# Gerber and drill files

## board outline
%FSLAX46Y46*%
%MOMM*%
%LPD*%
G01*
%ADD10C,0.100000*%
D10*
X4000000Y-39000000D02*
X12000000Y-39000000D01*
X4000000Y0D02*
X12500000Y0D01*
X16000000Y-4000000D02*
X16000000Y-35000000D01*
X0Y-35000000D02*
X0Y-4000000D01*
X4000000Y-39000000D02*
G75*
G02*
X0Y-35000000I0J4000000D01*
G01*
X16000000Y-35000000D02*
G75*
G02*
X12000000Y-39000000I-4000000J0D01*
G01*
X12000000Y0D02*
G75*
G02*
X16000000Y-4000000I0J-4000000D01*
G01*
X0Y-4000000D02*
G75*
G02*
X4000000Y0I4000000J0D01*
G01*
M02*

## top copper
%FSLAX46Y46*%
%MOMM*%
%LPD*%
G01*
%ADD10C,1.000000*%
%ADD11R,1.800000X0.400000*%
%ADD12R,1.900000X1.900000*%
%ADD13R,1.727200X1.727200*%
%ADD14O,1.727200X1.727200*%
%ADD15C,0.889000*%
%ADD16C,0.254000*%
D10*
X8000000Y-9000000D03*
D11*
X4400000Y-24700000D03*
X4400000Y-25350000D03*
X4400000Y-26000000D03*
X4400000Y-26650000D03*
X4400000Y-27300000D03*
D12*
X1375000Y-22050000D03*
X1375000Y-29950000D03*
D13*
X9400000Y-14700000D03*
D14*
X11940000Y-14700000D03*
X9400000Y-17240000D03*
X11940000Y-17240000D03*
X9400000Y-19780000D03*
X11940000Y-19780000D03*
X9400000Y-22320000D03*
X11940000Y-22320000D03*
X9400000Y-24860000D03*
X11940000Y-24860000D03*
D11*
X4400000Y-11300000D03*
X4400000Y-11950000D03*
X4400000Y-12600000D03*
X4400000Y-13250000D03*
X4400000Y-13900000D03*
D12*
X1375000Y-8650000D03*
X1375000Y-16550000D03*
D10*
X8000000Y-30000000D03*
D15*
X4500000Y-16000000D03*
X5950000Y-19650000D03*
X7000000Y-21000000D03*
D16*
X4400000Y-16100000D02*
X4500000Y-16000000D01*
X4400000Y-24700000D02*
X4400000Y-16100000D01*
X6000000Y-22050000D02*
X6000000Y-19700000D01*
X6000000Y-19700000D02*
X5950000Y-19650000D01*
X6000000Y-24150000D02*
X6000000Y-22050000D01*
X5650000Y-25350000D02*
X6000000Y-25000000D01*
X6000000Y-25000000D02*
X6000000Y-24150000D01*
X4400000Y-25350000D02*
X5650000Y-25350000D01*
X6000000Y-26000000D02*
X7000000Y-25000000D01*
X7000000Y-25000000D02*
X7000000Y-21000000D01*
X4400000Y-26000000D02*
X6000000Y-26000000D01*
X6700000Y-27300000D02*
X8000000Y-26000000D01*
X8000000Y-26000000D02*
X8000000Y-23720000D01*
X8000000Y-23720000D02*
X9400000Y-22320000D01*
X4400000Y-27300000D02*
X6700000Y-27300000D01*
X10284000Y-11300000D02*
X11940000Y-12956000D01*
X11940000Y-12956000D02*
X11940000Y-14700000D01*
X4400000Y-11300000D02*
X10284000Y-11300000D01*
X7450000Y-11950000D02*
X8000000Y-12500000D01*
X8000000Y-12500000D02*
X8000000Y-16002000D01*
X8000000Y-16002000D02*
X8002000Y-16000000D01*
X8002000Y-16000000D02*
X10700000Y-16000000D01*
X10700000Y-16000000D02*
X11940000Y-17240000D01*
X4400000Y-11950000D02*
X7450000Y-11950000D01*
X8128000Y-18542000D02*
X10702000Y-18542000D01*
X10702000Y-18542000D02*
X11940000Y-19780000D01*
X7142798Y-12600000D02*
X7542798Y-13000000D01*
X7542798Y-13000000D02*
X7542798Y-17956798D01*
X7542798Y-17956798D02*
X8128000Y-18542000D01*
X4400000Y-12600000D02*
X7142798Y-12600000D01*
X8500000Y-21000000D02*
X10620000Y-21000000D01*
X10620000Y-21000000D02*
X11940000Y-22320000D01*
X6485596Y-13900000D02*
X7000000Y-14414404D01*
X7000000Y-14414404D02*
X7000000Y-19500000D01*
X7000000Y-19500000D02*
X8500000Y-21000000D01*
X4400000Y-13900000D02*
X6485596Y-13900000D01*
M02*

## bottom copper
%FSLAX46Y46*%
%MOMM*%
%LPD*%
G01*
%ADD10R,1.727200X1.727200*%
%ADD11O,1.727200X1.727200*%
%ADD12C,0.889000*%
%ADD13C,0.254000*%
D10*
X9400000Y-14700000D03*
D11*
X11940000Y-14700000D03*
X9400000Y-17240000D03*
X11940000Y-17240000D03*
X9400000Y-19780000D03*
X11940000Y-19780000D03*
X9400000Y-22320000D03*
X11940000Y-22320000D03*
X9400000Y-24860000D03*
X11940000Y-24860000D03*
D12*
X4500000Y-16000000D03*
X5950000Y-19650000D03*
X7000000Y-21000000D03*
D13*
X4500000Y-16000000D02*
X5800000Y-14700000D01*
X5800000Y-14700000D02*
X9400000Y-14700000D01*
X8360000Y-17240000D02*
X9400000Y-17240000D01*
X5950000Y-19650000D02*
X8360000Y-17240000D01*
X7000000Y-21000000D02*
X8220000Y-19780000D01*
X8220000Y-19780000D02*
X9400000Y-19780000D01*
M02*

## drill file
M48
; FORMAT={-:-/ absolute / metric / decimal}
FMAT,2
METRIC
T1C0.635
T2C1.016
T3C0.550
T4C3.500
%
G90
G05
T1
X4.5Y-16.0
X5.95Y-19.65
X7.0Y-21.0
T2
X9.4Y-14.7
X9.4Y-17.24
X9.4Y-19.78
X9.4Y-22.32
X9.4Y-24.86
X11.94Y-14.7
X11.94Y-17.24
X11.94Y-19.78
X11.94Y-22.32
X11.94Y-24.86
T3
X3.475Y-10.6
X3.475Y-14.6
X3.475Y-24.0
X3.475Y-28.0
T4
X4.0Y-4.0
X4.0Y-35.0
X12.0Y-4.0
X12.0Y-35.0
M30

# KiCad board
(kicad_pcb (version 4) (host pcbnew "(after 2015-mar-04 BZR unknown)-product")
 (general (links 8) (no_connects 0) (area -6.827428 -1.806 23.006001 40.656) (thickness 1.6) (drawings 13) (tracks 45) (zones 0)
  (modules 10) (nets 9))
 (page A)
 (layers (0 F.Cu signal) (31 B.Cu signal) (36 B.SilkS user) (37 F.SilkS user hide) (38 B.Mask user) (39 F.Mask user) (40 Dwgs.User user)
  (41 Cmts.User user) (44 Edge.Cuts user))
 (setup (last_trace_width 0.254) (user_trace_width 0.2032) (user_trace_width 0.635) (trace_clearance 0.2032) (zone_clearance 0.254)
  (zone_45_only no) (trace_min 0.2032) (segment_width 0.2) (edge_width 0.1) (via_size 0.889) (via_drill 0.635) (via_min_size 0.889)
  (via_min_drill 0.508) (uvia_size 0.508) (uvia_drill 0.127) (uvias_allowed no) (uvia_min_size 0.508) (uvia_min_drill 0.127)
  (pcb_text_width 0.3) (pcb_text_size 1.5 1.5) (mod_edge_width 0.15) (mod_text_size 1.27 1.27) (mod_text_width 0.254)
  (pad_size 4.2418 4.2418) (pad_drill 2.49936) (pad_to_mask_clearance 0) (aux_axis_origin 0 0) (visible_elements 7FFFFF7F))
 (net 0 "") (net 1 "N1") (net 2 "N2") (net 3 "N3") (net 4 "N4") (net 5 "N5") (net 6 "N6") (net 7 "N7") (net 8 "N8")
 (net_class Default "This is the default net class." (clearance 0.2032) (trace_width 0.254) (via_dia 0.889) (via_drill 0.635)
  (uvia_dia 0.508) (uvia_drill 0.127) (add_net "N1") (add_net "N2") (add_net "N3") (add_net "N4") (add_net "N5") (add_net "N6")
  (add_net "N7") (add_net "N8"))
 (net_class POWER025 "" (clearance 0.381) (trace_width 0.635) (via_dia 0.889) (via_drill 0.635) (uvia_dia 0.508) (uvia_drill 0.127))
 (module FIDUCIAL (layer F.Cu) (at 8 9)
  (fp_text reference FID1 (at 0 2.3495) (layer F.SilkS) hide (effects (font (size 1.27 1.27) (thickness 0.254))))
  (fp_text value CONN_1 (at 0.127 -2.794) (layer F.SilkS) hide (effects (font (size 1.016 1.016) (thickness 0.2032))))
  (pad 1 smd circle (at 0 0) (size 1 1) (layers F.Cu F.Mask) (solder_mask_margin 1) (clearance 1)))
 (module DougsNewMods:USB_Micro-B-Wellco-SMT (layer F.Cu) (at 4 26 270)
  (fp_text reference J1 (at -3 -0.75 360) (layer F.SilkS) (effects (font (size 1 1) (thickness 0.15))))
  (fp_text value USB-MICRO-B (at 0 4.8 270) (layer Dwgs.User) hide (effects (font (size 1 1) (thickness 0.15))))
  (pad 1 smd rect (at -1.3 -0.4 270) (size 0.4 1.8) (layers F.Cu F.Mask) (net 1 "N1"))
  (pad 2 smd rect (at -0.65 -0.4 270) (size 0.4 1.8) (layers F.Cu F.Mask) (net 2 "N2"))
  (pad 3 smd rect (at 0 -0.4 270) (size 0.4 1.8) (layers F.Cu F.Mask) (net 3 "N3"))
  (pad 4 smd rect (at 0.65 -0.4 270) (size 0.4 1.8) (layers F.Cu F.Mask))
  (pad 5 smd rect (at 1.3 -0.4 270) (size 0.4 1.8) (layers F.Cu F.Mask) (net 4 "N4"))
  (pad "" np_thru_hole circle (at -2 0.525) (size 0.55 0.55) (drill 0.55) (layers *.Cu *.Mask F.SilkS))
  (pad "" np_thru_hole circle (at 2 0.525) (size 0.55 0.55) (drill oval 0.55) (layers *.Cu *.Mask F.SilkS))
  (pad 7 smd rect (at -3.95 2.625) (size 1.9 1.9) (layers F.Cu F.Mask))
  (pad 6 smd rect (at 3.95 2.625) (size 1.9 1.9) (layers F.Cu F.Mask)))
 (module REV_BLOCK (layer B.Cu) (at 13.15 10.8)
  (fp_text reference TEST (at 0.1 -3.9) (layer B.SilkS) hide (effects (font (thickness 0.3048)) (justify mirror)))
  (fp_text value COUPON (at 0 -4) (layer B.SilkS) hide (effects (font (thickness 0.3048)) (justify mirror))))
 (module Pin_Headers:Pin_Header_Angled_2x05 (layer F.Cu) (at 9.4 14.7)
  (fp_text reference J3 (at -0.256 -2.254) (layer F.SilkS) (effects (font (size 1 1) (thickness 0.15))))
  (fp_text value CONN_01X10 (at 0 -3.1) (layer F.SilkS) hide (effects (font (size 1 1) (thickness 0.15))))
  (pad 1 thru_hole rect (at 0 0) (size 1.7272 1.7272) (drill 1.016) (layers *.Cu *.Mask F.SilkS) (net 1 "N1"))
  (pad 2 thru_hole oval (at 2.54 0) (size 1.7272 1.7272) (drill 1.016) (layers *.Cu *.Mask F.SilkS) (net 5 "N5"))
  (pad 3 thru_hole oval (at 0 2.54) (size 1.7272 1.7272) (drill 1.016) (layers *.Cu *.Mask F.SilkS) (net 2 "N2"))
  (pad 4 thru_hole oval (at 2.54 2.54) (size 1.7272 1.7272) (drill 1.016) (layers *.Cu *.Mask F.SilkS) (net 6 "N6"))
  (pad 5 thru_hole oval (at 0 5.08) (size 1.7272 1.7272) (drill 1.016) (layers *.Cu *.Mask F.SilkS) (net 3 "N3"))
  (pad 6 thru_hole oval (at 2.54 5.08) (size 1.7272 1.7272) (drill 1.016) (layers *.Cu *.Mask F.SilkS) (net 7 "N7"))
  (pad 7 thru_hole oval (at 0 7.62) (size 1.7272 1.7272) (drill 1.016) (layers *.Cu *.Mask F.SilkS) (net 4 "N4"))
  (pad 8 thru_hole oval (at 2.54 7.62) (size 1.7272 1.7272) (drill 1.016) (layers *.Cu *.Mask F.SilkS) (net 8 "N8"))
  (pad 9 thru_hole oval (at 0 10.16) (size 1.7272 1.7272) (drill 1.016) (layers *.Cu *.Mask F.SilkS))
  (pad 10 thru_hole oval (at 2.54 10.16) (size 1.7272 1.7272) (drill 1.016) (layers *.Cu *.Mask F.SilkS)))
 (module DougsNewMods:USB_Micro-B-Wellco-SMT (layer F.Cu) (at 4 12.6 270) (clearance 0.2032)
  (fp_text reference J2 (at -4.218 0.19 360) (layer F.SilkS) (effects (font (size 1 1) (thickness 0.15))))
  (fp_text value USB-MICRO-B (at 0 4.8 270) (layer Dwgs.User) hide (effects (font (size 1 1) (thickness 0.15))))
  (pad 1 smd rect (at -1.3 -0.4 270) (size 0.4 1.8) (layers F.Cu F.Mask) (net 5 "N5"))
  (pad 2 smd rect (at -0.65 -0.4 270) (size 0.4 1.8) (layers F.Cu F.Mask) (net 6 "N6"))
  (pad 3 smd rect (at 0 -0.4 270) (size 0.4 1.8) (layers F.Cu F.Mask) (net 7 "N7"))
  (pad 4 smd rect (at 0.65 -0.4 270) (size 0.4 1.8) (layers F.Cu F.Mask))
  (pad 5 smd rect (at 1.3 -0.4 270) (size 0.4 1.8) (layers F.Cu F.Mask) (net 8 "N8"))
  (pad "" np_thru_hole circle (at -2 0.525) (size 0.55 0.55) (drill 0.55) (layers *.Cu *.Mask F.SilkS))
  (pad "" np_thru_hole circle (at 2 0.525) (size 0.55 0.55) (drill oval 0.55) (layers *.Cu *.Mask F.SilkS))
  (pad 7 smd rect (at -3.95 2.625) (size 1.9 1.9) (layers F.Cu F.Mask))
  (pad 6 smd rect (at 3.95 2.625) (size 1.9 1.9) (layers F.Cu F.Mask)))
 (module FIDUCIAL (layer F.Cu) (at 8 30)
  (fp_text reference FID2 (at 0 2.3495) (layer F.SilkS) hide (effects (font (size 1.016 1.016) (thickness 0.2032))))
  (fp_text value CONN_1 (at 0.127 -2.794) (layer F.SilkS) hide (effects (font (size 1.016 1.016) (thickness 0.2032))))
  (pad 1 smd circle (at 0 0) (size 1 1) (layers F.Cu F.Mask) (solder_mask_margin 1) (clearance 1)))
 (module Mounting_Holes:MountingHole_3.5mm (layer F.Cu) (at 4 4)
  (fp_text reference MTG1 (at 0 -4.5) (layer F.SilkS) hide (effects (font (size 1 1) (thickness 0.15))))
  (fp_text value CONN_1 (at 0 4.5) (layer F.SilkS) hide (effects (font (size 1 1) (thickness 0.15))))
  (pad 1 np_thru_hole circle (at 0 0) (size 3.5 3.5) (drill 3.5) (layers *.Cu *.Mask F.SilkS)))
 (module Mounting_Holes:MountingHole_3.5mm (layer F.Cu) (at 12 4)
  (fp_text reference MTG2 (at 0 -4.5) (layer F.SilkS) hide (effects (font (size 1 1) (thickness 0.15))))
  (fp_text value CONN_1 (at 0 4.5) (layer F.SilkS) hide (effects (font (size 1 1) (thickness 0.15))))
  (pad 1 np_thru_hole circle (at 0 0) (size 3.5 3.5) (drill 3.5) (layers *.Cu *.Mask F.SilkS)))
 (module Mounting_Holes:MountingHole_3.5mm (layer F.Cu) (at 4 35)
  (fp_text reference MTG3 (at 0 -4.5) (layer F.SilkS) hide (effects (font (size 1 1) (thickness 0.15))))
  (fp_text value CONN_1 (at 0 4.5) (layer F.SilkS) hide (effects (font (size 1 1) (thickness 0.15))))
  (pad 1 np_thru_hole circle (at 0 0) (size 3.5 3.5) (drill 3.5) (layers *.Cu *.Mask F.SilkS)))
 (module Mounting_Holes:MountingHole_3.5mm (layer F.Cu) (at 12 35)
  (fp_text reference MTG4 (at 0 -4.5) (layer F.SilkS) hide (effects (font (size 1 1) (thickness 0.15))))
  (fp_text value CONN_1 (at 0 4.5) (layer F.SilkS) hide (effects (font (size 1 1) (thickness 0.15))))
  (pad 1 np_thru_hole circle (at 0 0) (size 3.5 3.5) (drill 3.5) (layers *.Cu *.Mask F.SilkS)))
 (gr_line (start 4 39) (end 12 39) (angle 90) (layer Edge.Cuts) (width 0.1))
 (gr_line (start 4 0) (end 12.5 0) (angle 90) (layer Edge.Cuts) (width 0.1))
 (gr_line (start 16 4) (end 16 35) (angle 90) (layer Edge.Cuts) (width 0.1))
 (gr_line (start 0 35) (end 0 4) (angle 90) (layer Edge.Cuts) (width 0.1))
 (gr_arc (start 4 35) (end 4 39) (angle 90) (layer Edge.Cuts) (width 0.1))
 (gr_arc (start 12 35) (end 16 35) (angle 90) (layer Edge.Cuts) (width 0.1))
 (gr_arc (start 12 4) (end 12 0) (angle 90) (layer Edge.Cuts) (width 0.1))
 (gr_arc (start 4 4) (end 0 4) (angle 90) (layer Edge.Cuts) (width 0.1))
 (segment (start 4.4 16.1) (end 4.5 16) (width 0.254) (layer F.Cu) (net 1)) (via (at 4.5 16) (size 0.889) (layers F.Cu B.Cu) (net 1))
 (segment (start 4.5 16) (end 5.8 14.7) (width 0.254) (layer B.Cu) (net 1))
 (segment (start 5.8 14.7) (end 9.4 14.7) (width 0.254) (layer B.Cu) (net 1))
 (segment (start 4.4 24.7) (end 4.4 16.1) (width 0.254) (layer F.Cu) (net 1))
 (segment (start 6 22.05) (end 6 19.7) (width 0.254) (layer F.Cu) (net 2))
 (segment (start 8.36 17.24) (end 9.4 17.24) (width 0.254) (layer B.Cu) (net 2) (status 800000))
 (segment (start 5.95 19.65) (end 8.36 17.24) (width 0.254) (layer B.Cu) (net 2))
 (via (at 5.95 19.65) (size 0.889) (layers F.Cu B.Cu) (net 2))
 (segment (start 6 19.7) (end 5.95 19.65) (width 0.254) (layer F.Cu) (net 2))
 (segment (start 6 24.15) (end 6 22.05) (width 0.254) (layer F.Cu) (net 2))
 (segment (start 5.65 25.35) (end 6 25) (width 0.254) (layer F.Cu) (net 2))
 (segment (start 6 25) (end 6 24.15) (width 0.254) (layer F.Cu) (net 2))
 (segment (start 4.4 25.35) (end 5.65 25.35) (width 0.254) (layer F.Cu) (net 2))
 (segment (start 6 26) (end 7 25) (width 0.254) (layer F.Cu) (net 3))
 (segment (start 7 25) (end 7 21) (width 0.254) (layer F.Cu) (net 3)) (via (at 7 21) (size 0.889) (layers F.Cu B.Cu) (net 3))
 (segment (start 7 21) (end 8.22 19.78) (width 0.254) (layer B.Cu) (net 3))
 (segment (start 8.22 19.78) (end 9.4 19.78) (width 0.254) (layer B.Cu) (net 3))
 (segment (start 4.4 26) (end 6 26) (width 0.254) (layer F.Cu) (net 3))
 (segment (start 6.7 27.3) (end 8 26) (width 0.254) (layer F.Cu) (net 4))
 (segment (start 8 26) (end 8 23.72) (width 0.254) (layer F.Cu) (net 4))
 (segment (start 8 23.72) (end 9.4 22.32) (width 0.254) (layer F.Cu) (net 4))
 (segment (start 4.4 27.3) (end 6.7 27.3) (width 0.254) (layer F.Cu) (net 4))
 (segment (start 10.284 11.3) (end 11.94 12.956) (width 0.254) (layer F.Cu) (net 5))
 (segment (start 11.94 12.956) (end 11.94 14.7) (width 0.254) (layer F.Cu) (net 5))
 (segment (start 4.4 11.3) (end 10.284 11.3) (width 0.254) (layer F.Cu) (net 5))
 (segment (start 7.45 11.95) (end 8 12.5) (width 0.254) (layer F.Cu) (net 6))
 (segment (start 8 12.5) (end 8 16.002) (width 0.254) (layer F.Cu) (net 6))
 (segment (start 8 16.002) (end 8.002 16) (width 0.254) (layer F.Cu) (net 6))
 (segment (start 8.002 16) (end 10.7 16) (width 0.254) (layer F.Cu) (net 6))
 (segment (start 10.7 16) (end 11.94 17.24) (width 0.254) (layer F.Cu) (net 6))
 (segment (start 4.4 11.95) (end 7.45 11.95) (width 0.254) (layer F.Cu) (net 6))
 (segment (start 8.128 18.542) (end 10.702 18.542) (width 0.254) (layer F.Cu) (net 7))
 (segment (start 10.702 18.542) (end 11.94 19.78) (width 0.254) (layer F.Cu) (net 7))
 (segment (start 7.142798 12.6) (end 7.542798 13) (width 0.254) (layer F.Cu) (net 7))
 (segment (start 7.542798 13) (end 7.542798 17.956798) (width 0.254) (layer F.Cu) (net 7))
 (segment (start 7.542798 17.956798) (end 8.128 18.542) (width 0.254) (layer F.Cu) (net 7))
 (segment (start 4.4 12.6) (end 7.142798 12.6) (width 0.254) (layer F.Cu) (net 7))
 (segment (start 8.5 21) (end 10.62 21) (width 0.254) (layer F.Cu) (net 8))
 (segment (start 10.62 21) (end 11.94 22.32) (width 0.254) (layer F.Cu) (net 8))
 (segment (start 6.485596 13.9) (end 7 14.414404) (width 0.254) (layer F.Cu) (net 8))
 (segment (start 7 14.414404) (end 7 19.5) (width 0.254) (layer F.Cu) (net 8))
 (segment (start 7 19.5) (end 8.5 21) (width 0.254) (layer F.Cu) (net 8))
 (segment (start 4.4 13.9) (end 6.485596 13.9) (width 0.254) (layer F.Cu) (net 8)))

